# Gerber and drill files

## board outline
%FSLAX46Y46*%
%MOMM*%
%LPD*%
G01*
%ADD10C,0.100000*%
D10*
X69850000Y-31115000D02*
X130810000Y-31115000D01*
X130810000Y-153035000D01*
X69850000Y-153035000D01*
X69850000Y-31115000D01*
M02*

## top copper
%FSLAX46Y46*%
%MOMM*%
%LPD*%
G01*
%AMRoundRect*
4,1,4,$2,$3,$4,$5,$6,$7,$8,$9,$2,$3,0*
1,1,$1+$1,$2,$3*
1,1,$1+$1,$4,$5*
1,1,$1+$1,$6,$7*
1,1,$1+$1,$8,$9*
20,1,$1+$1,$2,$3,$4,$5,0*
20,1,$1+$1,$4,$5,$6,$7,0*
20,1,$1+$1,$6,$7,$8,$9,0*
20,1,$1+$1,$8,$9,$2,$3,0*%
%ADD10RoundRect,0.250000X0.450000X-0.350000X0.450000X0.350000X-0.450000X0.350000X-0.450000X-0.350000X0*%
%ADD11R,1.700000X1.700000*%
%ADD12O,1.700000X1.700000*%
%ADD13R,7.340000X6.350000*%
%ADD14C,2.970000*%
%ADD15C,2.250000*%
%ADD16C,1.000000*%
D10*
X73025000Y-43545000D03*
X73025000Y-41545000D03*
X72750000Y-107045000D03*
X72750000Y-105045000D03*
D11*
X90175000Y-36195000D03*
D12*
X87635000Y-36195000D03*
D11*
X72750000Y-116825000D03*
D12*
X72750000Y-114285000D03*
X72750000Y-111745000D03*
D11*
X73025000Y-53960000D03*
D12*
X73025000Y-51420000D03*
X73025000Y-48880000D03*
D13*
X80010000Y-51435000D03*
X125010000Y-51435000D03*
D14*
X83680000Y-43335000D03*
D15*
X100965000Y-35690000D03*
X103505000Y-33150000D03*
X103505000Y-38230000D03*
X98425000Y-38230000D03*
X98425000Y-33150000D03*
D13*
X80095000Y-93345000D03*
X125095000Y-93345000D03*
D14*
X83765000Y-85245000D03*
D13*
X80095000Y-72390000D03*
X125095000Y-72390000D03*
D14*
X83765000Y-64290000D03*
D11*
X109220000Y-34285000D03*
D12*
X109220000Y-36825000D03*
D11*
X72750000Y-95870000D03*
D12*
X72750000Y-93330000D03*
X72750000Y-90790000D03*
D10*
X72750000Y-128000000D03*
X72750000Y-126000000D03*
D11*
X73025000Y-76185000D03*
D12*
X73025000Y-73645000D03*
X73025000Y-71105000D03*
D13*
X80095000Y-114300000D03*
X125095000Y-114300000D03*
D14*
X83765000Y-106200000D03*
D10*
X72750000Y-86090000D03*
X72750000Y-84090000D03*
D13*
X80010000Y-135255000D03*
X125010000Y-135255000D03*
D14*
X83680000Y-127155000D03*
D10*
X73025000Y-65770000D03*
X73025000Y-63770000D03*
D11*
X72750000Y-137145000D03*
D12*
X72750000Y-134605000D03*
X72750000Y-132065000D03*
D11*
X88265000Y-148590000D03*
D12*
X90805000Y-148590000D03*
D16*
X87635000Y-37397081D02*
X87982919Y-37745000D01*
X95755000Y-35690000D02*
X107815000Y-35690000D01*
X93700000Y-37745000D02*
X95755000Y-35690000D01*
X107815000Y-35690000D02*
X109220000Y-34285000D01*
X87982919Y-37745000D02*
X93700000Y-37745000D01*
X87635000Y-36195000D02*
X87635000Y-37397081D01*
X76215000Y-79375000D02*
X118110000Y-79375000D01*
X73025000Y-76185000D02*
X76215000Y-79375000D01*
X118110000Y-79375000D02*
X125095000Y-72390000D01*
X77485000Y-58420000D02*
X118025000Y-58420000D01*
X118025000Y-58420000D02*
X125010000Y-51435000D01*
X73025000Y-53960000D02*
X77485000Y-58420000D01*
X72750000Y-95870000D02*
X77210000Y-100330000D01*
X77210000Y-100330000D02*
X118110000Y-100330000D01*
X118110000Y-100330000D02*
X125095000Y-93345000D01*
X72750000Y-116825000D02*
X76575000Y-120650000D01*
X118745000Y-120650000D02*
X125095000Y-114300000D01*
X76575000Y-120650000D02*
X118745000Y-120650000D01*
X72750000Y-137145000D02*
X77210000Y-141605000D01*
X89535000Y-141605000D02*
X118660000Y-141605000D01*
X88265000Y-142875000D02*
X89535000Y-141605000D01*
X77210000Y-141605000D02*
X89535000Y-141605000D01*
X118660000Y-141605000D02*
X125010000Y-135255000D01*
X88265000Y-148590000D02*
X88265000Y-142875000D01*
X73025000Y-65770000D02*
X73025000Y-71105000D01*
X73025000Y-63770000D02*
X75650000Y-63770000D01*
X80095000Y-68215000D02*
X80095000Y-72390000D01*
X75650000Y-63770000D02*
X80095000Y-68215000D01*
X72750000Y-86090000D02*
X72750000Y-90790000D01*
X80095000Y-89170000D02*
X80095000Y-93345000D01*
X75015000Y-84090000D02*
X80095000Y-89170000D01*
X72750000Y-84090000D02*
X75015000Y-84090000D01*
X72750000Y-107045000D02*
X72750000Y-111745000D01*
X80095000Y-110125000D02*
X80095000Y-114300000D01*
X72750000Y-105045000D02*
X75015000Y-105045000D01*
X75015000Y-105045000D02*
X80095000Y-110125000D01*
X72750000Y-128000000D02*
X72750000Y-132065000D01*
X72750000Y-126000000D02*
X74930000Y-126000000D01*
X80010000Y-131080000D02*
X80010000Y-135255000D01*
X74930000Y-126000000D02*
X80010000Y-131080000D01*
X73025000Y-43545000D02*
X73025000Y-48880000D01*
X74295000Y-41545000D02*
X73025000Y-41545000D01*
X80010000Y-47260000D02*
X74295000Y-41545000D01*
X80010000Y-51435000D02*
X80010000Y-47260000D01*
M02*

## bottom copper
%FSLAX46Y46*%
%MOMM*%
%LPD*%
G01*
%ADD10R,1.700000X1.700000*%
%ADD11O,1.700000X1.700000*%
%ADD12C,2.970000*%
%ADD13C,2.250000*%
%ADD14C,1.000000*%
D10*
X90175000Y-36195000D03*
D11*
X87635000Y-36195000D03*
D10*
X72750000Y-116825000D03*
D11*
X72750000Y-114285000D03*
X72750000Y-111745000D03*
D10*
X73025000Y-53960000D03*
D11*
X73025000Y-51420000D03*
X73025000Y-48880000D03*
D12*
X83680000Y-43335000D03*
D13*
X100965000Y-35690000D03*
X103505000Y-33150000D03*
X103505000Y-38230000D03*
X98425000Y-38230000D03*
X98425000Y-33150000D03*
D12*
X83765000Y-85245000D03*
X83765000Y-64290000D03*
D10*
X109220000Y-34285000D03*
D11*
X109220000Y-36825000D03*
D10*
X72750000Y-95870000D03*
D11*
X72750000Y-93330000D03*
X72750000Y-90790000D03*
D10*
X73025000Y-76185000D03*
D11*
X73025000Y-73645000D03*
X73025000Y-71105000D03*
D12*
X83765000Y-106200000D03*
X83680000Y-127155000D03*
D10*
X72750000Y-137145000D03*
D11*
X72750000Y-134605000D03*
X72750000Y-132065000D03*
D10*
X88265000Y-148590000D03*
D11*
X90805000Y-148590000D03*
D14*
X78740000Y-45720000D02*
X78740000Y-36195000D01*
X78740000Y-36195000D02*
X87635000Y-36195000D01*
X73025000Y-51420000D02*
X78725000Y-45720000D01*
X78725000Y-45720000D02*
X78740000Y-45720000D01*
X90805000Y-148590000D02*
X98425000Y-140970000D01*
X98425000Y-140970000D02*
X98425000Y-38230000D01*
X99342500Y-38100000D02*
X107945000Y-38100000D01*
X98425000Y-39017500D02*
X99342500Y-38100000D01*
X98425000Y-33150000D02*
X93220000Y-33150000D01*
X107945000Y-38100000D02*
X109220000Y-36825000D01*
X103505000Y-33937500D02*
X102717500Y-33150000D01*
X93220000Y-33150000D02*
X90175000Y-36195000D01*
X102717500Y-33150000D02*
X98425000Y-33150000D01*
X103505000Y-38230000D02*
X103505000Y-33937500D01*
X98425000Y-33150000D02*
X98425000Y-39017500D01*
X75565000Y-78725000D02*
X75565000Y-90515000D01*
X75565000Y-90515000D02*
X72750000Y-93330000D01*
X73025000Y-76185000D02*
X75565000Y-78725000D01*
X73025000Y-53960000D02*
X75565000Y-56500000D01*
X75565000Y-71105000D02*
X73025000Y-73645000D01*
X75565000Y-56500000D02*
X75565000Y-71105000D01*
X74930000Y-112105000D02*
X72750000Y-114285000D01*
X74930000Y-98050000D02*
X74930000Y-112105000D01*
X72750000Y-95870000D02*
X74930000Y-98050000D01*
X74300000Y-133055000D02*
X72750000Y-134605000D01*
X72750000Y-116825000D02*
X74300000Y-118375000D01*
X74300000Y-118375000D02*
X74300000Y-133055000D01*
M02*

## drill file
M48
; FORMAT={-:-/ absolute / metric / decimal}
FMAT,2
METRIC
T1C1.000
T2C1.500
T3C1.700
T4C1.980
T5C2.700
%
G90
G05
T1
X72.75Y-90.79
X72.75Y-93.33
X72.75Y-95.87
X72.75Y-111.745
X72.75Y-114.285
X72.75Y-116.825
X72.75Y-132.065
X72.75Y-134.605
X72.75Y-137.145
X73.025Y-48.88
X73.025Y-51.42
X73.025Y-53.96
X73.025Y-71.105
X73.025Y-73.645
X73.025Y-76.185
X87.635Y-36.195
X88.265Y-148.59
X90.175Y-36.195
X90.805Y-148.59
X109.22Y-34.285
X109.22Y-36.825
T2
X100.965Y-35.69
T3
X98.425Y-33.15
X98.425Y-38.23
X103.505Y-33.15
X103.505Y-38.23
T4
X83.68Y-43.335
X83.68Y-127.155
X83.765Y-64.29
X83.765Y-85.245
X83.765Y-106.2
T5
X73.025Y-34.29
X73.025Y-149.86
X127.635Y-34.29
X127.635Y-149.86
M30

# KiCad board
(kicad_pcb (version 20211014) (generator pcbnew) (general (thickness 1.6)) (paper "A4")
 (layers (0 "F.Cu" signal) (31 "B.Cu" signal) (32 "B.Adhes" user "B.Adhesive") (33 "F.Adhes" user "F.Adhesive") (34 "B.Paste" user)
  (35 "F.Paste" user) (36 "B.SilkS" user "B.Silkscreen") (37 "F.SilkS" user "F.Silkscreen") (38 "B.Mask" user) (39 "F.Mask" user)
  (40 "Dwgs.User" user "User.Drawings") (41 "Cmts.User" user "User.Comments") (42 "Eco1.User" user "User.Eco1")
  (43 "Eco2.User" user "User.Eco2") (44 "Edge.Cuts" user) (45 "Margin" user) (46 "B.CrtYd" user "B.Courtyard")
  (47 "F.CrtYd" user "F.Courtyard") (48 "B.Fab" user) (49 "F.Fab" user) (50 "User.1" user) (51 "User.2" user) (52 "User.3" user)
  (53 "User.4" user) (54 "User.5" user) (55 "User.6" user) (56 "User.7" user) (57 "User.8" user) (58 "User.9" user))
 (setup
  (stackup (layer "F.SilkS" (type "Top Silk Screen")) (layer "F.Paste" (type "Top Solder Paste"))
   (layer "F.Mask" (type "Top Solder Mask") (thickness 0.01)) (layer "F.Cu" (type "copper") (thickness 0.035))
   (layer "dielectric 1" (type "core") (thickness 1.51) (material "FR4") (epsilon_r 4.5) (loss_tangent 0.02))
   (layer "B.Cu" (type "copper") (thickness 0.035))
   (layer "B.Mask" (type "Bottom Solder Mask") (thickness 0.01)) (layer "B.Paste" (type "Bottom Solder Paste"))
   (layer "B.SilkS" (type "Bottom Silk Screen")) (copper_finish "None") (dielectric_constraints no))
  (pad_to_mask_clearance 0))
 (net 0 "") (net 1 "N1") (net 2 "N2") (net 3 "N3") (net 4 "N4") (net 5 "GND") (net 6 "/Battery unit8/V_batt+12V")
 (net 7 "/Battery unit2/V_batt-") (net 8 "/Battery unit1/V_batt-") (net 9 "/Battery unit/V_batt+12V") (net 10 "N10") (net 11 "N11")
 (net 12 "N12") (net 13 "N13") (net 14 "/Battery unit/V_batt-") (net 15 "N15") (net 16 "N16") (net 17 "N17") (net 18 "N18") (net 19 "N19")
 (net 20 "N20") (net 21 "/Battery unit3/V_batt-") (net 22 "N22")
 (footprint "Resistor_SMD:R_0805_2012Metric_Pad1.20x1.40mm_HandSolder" (layer "F.Cu") (at 73.025 42.545 90)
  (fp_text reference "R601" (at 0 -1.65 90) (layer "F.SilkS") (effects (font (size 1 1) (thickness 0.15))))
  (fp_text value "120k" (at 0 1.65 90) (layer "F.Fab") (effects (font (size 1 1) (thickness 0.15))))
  (pad "1" smd roundrect (at -1 0 90) (size 1.2 1.4) (layers "F.Cu" "F.Paste" "F.Mask") (roundrect_rratio 0.208333) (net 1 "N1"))
  (pad "2" smd roundrect (at 1 0 90) (size 1.2 1.4) (layers "F.Cu" "F.Paste" "F.Mask") (roundrect_rratio 0.208333) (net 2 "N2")))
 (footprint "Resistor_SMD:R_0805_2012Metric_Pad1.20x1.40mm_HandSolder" (layer "F.Cu") (at 72.75 106.045 90)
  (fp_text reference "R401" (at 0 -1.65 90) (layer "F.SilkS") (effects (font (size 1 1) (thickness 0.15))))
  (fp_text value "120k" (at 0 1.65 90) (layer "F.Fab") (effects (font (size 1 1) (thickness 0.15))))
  (pad "1" smd roundrect (at -1 0 90) (size 1.2 1.4) (layers "F.Cu" "F.Paste" "F.Mask") (roundrect_rratio 0.208333) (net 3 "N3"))
  (pad "2" smd roundrect (at 1 0 90) (size 1.2 1.4) (layers "F.Cu" "F.Paste" "F.Mask") (roundrect_rratio 0.208333) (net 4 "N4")))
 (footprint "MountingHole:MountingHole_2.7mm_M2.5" (layer "F.Cu") (at 127.635 149.86 180)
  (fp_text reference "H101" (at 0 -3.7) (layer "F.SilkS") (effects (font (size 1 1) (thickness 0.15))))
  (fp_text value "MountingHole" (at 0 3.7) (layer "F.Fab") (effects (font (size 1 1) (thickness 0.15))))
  (pad "" np_thru_hole circle (at 0 0 180) (size 2.7 2.7) (drill 2.7) (layers *.Cu *.Mask)))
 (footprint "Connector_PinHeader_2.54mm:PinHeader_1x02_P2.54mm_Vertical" (layer "F.Cu") (at 90.175 36.195 -90)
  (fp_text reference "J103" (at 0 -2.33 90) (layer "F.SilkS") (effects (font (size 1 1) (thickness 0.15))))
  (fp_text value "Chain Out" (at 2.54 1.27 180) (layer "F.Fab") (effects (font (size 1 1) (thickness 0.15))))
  (pad "1" thru_hole rect (at 0 0 270) (size 1.7 1.7) (drill 1) (layers *.Cu *.Mask) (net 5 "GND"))
  (pad "2" thru_hole oval (at 0 2.54 270) (size 1.7 1.7) (drill 1) (layers *.Cu *.Mask) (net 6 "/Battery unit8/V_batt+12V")))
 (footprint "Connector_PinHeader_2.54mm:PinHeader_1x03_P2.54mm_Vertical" (layer "F.Cu") (at 72.75 116.825 180)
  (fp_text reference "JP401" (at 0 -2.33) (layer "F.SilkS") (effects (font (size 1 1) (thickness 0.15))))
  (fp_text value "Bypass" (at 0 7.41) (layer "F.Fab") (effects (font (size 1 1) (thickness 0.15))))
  (pad "1" thru_hole rect (at 0 0 180) (size 1.7 1.7) (drill 1) (layers *.Cu *.Mask) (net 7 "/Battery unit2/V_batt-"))
  (pad "2" thru_hole oval (at 0 2.54 180) (size 1.7 1.7) (drill 1) (layers *.Cu *.Mask) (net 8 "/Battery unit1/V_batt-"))
  (pad "3" thru_hole oval (at 0 5.08 180) (size 1.7 1.7) (drill 1) (layers *.Cu *.Mask) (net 3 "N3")))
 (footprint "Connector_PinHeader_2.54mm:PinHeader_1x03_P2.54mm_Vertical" (layer "F.Cu") (at 73.025 53.96 180)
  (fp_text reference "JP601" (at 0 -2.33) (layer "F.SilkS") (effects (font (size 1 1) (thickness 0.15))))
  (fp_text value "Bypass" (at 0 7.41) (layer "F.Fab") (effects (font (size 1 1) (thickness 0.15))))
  (pad "1" thru_hole rect (at 0 0 180) (size 1.7 1.7) (drill 1) (layers *.Cu *.Mask) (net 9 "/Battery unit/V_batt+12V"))
  (pad "2" thru_hole oval (at 0 2.54 180) (size 1.7 1.7) (drill 1) (layers *.Cu *.Mask) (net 6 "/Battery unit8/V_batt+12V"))
  (pad "3" thru_hole oval (at 0 5.08 180) (size 1.7 1.7) (drill 1) (layers *.Cu *.Mask) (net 1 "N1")))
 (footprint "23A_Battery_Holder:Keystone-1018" (layer "F.Cu") (at 102.51 51.435)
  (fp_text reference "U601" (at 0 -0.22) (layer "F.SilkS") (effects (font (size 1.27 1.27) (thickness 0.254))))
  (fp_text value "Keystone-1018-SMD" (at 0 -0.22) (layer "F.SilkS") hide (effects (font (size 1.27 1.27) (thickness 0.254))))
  (pad "1" smd rect (at -22.5 0 90) (size 6.35 7.34) (layers "F.Cu" "F.Paste" "F.Mask") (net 2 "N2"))
  (pad "2" smd rect (at 22.5 0 90) (size 6.35 7.34) (layers "F.Cu" "F.Paste" "F.Mask") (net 9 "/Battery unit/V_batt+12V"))
  (pad "MH1" thru_hole circle (at -18.83 -8.1) (size 2.97 2.97) (drill 1.98) (layers *.Cu *.Mask) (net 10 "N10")))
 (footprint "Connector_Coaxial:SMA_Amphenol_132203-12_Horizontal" (layer "F.Cu") (at 100.965 35.69)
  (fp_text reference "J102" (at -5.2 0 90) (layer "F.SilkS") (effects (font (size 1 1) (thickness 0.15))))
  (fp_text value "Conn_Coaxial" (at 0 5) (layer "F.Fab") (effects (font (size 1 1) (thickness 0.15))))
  (pad "1" thru_hole circle (at 0 0) (size 2.25 2.25) (drill 1.5) (layers *.Cu *.Mask) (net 6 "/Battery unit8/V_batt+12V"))
  (pad "2" thru_hole circle (at 2.54 -2.54) (size 2.25 2.25) (drill 1.7) (layers *.Cu *.Mask) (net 5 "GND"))
  (pad "2" thru_hole circle (at 2.54 2.54 90) (size 2.25 2.25) (drill 1.7) (layers *.Cu *.Mask) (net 5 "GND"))
  (pad "2" thru_hole circle (at -2.54 2.54) (size 2.25 2.25) (drill 1.7) (layers *.Cu *.Mask) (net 5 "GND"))
  (pad "2" thru_hole circle (at -2.54 -2.54) (size 2.25 2.25) (drill 1.7) (layers *.Cu *.Mask) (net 5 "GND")))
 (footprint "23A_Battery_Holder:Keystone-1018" (layer "F.Cu") (at 102.595 93.345)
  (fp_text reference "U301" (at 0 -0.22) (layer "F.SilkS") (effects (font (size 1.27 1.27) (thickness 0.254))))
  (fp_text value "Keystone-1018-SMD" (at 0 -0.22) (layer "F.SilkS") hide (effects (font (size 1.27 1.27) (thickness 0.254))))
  (pad "1" smd rect (at -22.5 0 90) (size 6.35 7.34) (layers "F.Cu" "F.Paste" "F.Mask") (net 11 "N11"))
  (pad "2" smd rect (at 22.5 0 90) (size 6.35 7.34) (layers "F.Cu" "F.Paste" "F.Mask") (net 8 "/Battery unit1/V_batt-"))
  (pad "MH1" thru_hole circle (at -18.83 -8.1) (size 2.97 2.97) (drill 1.98) (layers *.Cu *.Mask) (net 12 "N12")))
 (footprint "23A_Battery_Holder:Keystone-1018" (layer "F.Cu") (at 102.595 72.39)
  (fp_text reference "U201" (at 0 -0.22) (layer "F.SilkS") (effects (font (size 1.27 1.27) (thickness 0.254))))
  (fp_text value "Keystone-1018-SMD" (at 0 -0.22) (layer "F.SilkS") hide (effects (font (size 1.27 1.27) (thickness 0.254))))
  (pad "1" smd rect (at -22.5 0 90) (size 6.35 7.34) (layers "F.Cu" "F.Paste" "F.Mask") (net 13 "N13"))
  (pad "2" smd rect (at 22.5 0 90) (size 6.35 7.34) (layers "F.Cu" "F.Paste" "F.Mask") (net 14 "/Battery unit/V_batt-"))
  (pad "MH1" thru_hole circle (at -18.83 -8.1) (size 2.97 2.97) (drill 1.98) (layers *.Cu *.Mask) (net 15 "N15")))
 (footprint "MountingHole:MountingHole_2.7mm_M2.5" (layer "F.Cu") (at 73.025 34.29)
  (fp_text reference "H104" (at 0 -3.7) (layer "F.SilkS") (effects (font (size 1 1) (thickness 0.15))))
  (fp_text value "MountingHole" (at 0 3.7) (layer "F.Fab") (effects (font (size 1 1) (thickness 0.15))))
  (pad "" np_thru_hole circle (at 0 0) (size 2.7 2.7) (drill 2.7) (layers *.Cu *.Mask)))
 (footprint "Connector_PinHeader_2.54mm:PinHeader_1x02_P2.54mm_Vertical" (layer "F.Cu") (at 109.22 34.285)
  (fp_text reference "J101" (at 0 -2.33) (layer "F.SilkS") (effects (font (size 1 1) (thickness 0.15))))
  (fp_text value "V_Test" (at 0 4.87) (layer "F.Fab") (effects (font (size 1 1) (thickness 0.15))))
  (pad "1" thru_hole rect (at 0 0) (size 1.7 1.7) (drill 1) (layers *.Cu *.Mask) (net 6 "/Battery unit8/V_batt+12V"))
  (pad "2" thru_hole oval (at 0 2.54) (size 1.7 1.7) (drill 1) (layers *.Cu *.Mask) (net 5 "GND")))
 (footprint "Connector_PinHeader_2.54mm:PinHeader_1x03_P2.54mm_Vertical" (layer "F.Cu") (at 72.75 95.87 180)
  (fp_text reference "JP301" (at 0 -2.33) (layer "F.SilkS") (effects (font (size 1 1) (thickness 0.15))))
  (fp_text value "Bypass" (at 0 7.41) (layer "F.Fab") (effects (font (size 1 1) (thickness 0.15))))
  (pad "1" thru_hole rect (at 0 0 180) (size 1.7 1.7) (drill 1) (layers *.Cu *.Mask) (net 8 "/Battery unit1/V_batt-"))
  (pad "2" thru_hole oval (at 0 2.54 180) (size 1.7 1.7) (drill 1) (layers *.Cu *.Mask) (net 14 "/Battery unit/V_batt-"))
  (pad "3" thru_hole oval (at 0 5.08 180) (size 1.7 1.7) (drill 1) (layers *.Cu *.Mask) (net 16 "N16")))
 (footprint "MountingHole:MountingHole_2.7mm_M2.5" (layer "F.Cu") (at 73.025 149.86)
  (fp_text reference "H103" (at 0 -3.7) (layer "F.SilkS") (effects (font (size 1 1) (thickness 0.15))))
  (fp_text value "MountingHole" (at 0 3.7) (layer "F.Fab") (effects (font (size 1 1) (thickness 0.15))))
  (pad "" np_thru_hole circle (at 0 0) (size 2.7 2.7) (drill 2.7) (layers *.Cu *.Mask)))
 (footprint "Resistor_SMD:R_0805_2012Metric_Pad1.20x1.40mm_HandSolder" (layer "F.Cu") (at 72.75 127 90)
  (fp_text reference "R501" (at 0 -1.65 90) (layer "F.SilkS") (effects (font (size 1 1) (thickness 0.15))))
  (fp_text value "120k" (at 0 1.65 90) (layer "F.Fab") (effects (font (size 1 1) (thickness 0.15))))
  (pad "1" smd roundrect (at -1 0 90) (size 1.2 1.4) (layers "F.Cu" "F.Paste" "F.Mask") (roundrect_rratio 0.208333) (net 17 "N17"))
  (pad "2" smd roundrect (at 1 0 90) (size 1.2 1.4) (layers "F.Cu" "F.Paste" "F.Mask") (roundrect_rratio 0.208333) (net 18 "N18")))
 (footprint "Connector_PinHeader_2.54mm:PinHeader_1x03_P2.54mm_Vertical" (layer "F.Cu") (at 73.025 76.185 180)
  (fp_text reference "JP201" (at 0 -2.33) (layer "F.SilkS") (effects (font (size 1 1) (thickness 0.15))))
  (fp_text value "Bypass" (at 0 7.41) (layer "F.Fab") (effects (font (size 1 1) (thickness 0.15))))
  (pad "1" thru_hole rect (at 0 0 180) (size 1.7 1.7) (drill 1) (layers *.Cu *.Mask) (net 14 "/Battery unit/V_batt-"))
  (pad "2" thru_hole oval (at 0 2.54 180) (size 1.7 1.7) (drill 1) (layers *.Cu *.Mask) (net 9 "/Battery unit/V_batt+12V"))
  (pad "3" thru_hole oval (at 0 5.08 180) (size 1.7 1.7) (drill 1) (layers *.Cu *.Mask) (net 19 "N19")))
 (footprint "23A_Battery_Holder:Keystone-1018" (layer "F.Cu") (at 102.595 114.3)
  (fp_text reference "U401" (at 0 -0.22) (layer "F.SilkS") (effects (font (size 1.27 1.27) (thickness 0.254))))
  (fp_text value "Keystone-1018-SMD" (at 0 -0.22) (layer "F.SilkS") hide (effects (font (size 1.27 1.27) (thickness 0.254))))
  (pad "1" smd rect (at -22.5 0 90) (size 6.35 7.34) (layers "F.Cu" "F.Paste" "F.Mask") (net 4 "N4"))
  (pad "2" smd rect (at 22.5 0 90) (size 6.35 7.34) (layers "F.Cu" "F.Paste" "F.Mask") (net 7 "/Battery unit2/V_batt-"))
  (pad "MH1" thru_hole circle (at -18.83 -8.1) (size 2.97 2.97) (drill 1.98) (layers *.Cu *.Mask) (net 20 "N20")))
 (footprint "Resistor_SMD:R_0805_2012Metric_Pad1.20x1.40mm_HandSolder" (layer "F.Cu") (at 72.75 85.09 90)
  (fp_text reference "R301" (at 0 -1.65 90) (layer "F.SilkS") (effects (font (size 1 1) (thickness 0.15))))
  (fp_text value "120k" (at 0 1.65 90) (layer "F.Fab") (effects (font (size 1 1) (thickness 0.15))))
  (pad "1" smd roundrect (at -1 0 90) (size 1.2 1.4) (layers "F.Cu" "F.Paste" "F.Mask") (roundrect_rratio 0.208333) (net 16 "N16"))
  (pad "2" smd roundrect (at 1 0 90) (size 1.2 1.4) (layers "F.Cu" "F.Paste" "F.Mask") (roundrect_rratio 0.208333) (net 11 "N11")))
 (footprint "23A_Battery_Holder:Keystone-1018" (layer "F.Cu") (at 102.51 135.255)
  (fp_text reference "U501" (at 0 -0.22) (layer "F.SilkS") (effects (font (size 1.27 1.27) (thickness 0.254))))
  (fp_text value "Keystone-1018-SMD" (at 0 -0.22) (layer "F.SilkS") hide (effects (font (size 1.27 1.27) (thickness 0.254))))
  (pad "1" smd rect (at -22.5 0 90) (size 6.35 7.34) (layers "F.Cu" "F.Paste" "F.Mask") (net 18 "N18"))
  (pad "2" smd rect (at 22.5 0 90) (size 6.35 7.34) (layers "F.Cu" "F.Paste" "F.Mask") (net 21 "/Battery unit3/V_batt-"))
  (pad "MH1" thru_hole circle (at -18.83 -8.1) (size 2.97 2.97) (drill 1.98) (layers *.Cu *.Mask) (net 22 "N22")))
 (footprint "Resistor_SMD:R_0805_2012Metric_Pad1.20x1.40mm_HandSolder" (layer "F.Cu") (at 73.025 64.77 90)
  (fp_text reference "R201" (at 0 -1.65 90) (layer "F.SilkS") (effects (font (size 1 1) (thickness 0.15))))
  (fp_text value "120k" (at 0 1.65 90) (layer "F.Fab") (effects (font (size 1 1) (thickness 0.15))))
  (pad "1" smd roundrect (at -1 0 90) (size 1.2 1.4) (layers "F.Cu" "F.Paste" "F.Mask") (roundrect_rratio 0.208333) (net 19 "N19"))
  (pad "2" smd roundrect (at 1 0 90) (size 1.2 1.4) (layers "F.Cu" "F.Paste" "F.Mask") (roundrect_rratio 0.208333) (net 13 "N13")))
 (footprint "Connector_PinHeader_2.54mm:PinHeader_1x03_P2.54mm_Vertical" (layer "F.Cu") (at 72.75 137.145 180)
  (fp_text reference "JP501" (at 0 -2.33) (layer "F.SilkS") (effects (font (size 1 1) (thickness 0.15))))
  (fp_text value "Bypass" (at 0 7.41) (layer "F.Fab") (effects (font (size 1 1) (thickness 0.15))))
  (pad "1" thru_hole rect (at 0 0 180) (size 1.7 1.7) (drill 1) (layers *.Cu *.Mask) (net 21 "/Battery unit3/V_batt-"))
  (pad "2" thru_hole oval (at 0 2.54 180) (size 1.7 1.7) (drill 1) (layers *.Cu *.Mask) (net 7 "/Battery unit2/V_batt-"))
  (pad "3" thru_hole oval (at 0 5.08 180) (size 1.7 1.7) (drill 1) (layers *.Cu *.Mask) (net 17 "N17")))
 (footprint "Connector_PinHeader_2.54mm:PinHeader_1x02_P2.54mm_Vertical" (layer "F.Cu") (at 88.265 148.59 90)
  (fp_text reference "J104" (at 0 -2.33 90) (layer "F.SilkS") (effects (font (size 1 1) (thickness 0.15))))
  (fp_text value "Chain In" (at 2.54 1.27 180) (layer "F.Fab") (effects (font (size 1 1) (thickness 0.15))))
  (pad "1" thru_hole rect (at 0 0 90) (size 1.7 1.7) (drill 1) (layers *.Cu *.Mask) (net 21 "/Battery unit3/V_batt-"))
  (pad "2" thru_hole oval (at 0 2.54 90) (size 1.7 1.7) (drill 1) (layers *.Cu *.Mask) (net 5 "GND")))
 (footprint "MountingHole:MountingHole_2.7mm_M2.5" (layer "F.Cu") (at 127.635 34.29 180)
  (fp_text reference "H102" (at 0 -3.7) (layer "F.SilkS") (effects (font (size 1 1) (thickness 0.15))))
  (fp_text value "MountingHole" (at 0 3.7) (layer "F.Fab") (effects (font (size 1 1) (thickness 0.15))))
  (pad "" np_thru_hole circle (at 0 0 180) (size 2.7 2.7) (drill 2.7) (layers *.Cu *.Mask)))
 (gr_rect (start 69.85 31.115) (end 130.81 153.035) (layer "Edge.Cuts") (width 0.1) (fill none))
 (segment (start 87.635 37.397081) (end 87.982919 37.745) (width 1) (layer "F.Cu") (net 6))
 (segment (start 95.755 35.69) (end 107.815 35.69) (width 1) (layer "F.Cu") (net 6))
 (segment (start 93.7 37.745) (end 95.755 35.69) (width 1) (layer "F.Cu") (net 6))
 (segment (start 107.815 35.69) (end 109.22 34.285) (width 1) (layer "F.Cu") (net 6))
 (segment (start 87.982919 37.745) (end 93.7 37.745) (width 1) (layer "F.Cu") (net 6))
 (segment (start 87.635 36.195) (end 87.635 37.397081) (width 1) (layer "F.Cu") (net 6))
 (segment (start 78.74 45.72) (end 78.74 36.195) (width 1) (layer "B.Cu") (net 6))
 (segment (start 78.74 36.195) (end 87.635 36.195) (width 1) (layer "B.Cu") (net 6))
 (segment (start 73.025 51.42) (end 78.725 45.72) (width 1) (layer "B.Cu") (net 6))
 (segment (start 78.725 45.72) (end 78.74 45.72) (width 1) (layer "B.Cu") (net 6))
 (segment (start 90.805 148.59) (end 98.425 140.97) (width 1) (layer "B.Cu") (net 5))
 (segment (start 98.425 140.97) (end 98.425 38.23) (width 1) (layer "B.Cu") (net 5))
 (segment (start 99.3425 38.1) (end 107.945 38.1) (width 1) (layer "B.Cu") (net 5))
 (segment (start 98.425 39.0175) (end 99.3425 38.1) (width 1) (layer "B.Cu") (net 5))
 (segment (start 98.425 33.15) (end 93.22 33.15) (width 1) (layer "B.Cu") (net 5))
 (segment (start 107.945 38.1) (end 109.22 36.825) (width 1) (layer "B.Cu") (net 5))
 (segment (start 103.505 33.9375) (end 102.7175 33.15) (width 1) (layer "B.Cu") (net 5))
 (segment (start 93.22 33.15) (end 90.175 36.195) (width 1) (layer "B.Cu") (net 5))
 (segment (start 102.7175 33.15) (end 98.425 33.15) (width 1) (layer "B.Cu") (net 5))
 (segment (start 103.505 38.23) (end 103.505 33.9375) (width 1) (layer "B.Cu") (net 5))
 (segment (start 98.425 33.15) (end 98.425 39.0175) (width 1) (layer "B.Cu") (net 5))
 (segment (start 76.215 79.375) (end 118.11 79.375) (width 1) (layer "F.Cu") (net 14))
 (segment (start 73.025 76.185) (end 76.215 79.375) (width 1) (layer "F.Cu") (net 14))
 (segment (start 118.11 79.375) (end 125.095 72.39) (width 1) (layer "F.Cu") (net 14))
 (segment (start 75.565 78.725) (end 75.565 90.515) (width 1) (layer "B.Cu") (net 14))
 (segment (start 75.565 90.515) (end 72.75 93.33) (width 1) (layer "B.Cu") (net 14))
 (segment (start 73.025 76.185) (end 75.565 78.725) (width 1) (layer "B.Cu") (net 14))
 (segment (start 77.485 58.42) (end 118.025 58.42) (width 1) (layer "F.Cu") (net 9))
 (segment (start 118.025 58.42) (end 125.01 51.435) (width 1) (layer "F.Cu") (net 9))
 (segment (start 73.025 53.96) (end 77.485 58.42) (width 1) (layer "F.Cu") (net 9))
 (segment (start 73.025 53.96) (end 75.565 56.5) (width 1) (layer "B.Cu") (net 9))
 (segment (start 75.565 71.105) (end 73.025 73.645) (width 1) (layer "B.Cu") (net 9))
 (segment (start 75.565 56.5) (end 75.565 71.105) (width 1) (layer "B.Cu") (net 9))
 (segment (start 72.75 95.87) (end 77.21 100.33) (width 1) (layer "F.Cu") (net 8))
 (segment (start 77.21 100.33) (end 118.11 100.33) (width 1) (layer "F.Cu") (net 8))
 (segment (start 118.11 100.33) (end 125.095 93.345) (width 1) (layer "F.Cu") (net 8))
 (segment (start 74.93 112.105) (end 72.75 114.285) (width 1) (layer "B.Cu") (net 8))
 (segment (start 74.93 98.05) (end 74.93 112.105) (width 1) (layer "B.Cu") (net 8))
 (segment (start 72.75 95.87) (end 74.93 98.05) (width 1) (layer "B.Cu") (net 8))
 (segment (start 72.75 116.825) (end 76.575 120.65) (width 1) (layer "F.Cu") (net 7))
 (segment (start 118.745 120.65) (end 125.095 114.3) (width 1) (layer "F.Cu") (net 7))
 (segment (start 76.575 120.65) (end 118.745 120.65) (width 1) (layer "F.Cu") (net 7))
 (segment (start 74.3 133.055) (end 72.75 134.605) (width 1) (layer "B.Cu") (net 7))
 (segment (start 72.75 116.825) (end 74.3 118.375) (width 1) (layer "B.Cu") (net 7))
 (segment (start 74.3 118.375) (end 74.3 133.055) (width 1) (layer "B.Cu") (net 7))
 (segment (start 72.75 137.145) (end 77.21 141.605) (width 1) (layer "F.Cu") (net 21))
 (segment (start 89.535 141.605) (end 118.66 141.605) (width 1) (layer "F.Cu") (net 21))
 (segment (start 88.265 142.875) (end 89.535 141.605) (width 1) (layer "F.Cu") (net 21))
 (segment (start 77.21 141.605) (end 89.535 141.605) (width 1) (layer "F.Cu") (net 21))
 (segment (start 118.66 141.605) (end 125.01 135.255) (width 1) (layer "F.Cu") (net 21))
 (segment (start 88.265 148.59) (end 88.265 142.875) (width 1) (layer "F.Cu") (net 21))
 (segment (start 73.025 65.77) (end 73.025 71.105) (width 1) (layer "F.Cu") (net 19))
 (segment (start 73.025 63.77) (end 75.65 63.77) (width 1) (layer "F.Cu") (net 13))
 (segment (start 80.095 68.215) (end 80.095 72.39) (width 1) (layer "F.Cu") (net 13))
 (segment (start 75.65 63.77) (end 80.095 68.215) (width 1) (layer "F.Cu") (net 13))
 (segment (start 72.75 86.09) (end 72.75 90.79) (width 1) (layer "F.Cu") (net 16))
 (segment (start 80.095 89.17) (end 80.095 93.345) (width 1) (layer "F.Cu") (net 11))
 (segment (start 75.015 84.09) (end 80.095 89.17) (width 1) (layer "F.Cu") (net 11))
 (segment (start 72.75 84.09) (end 75.015 84.09) (width 1) (layer "F.Cu") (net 11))
 (segment (start 72.75 107.045) (end 72.75 111.745) (width 1) (layer "F.Cu") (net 3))
 (segment (start 80.095 110.125) (end 80.095 114.3) (width 1) (layer "F.Cu") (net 4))
 (segment (start 72.75 105.045) (end 75.015 105.045) (width 1) (layer "F.Cu") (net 4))
 (segment (start 75.015 105.045) (end 80.095 110.125) (width 1) (layer "F.Cu") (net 4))
 (segment (start 72.75 128) (end 72.75 132.065) (width 1) (layer "F.Cu") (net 17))
 (segment (start 72.75 126) (end 74.93 126) (width 1) (layer "F.Cu") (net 18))
 (segment (start 80.01 131.08) (end 80.01 135.255) (width 1) (layer "F.Cu") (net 18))
 (segment (start 74.93 126) (end 80.01 131.08) (width 1) (layer "F.Cu") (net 18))
 (segment (start 73.025 43.545) (end 73.025 48.88) (width 1) (layer "F.Cu") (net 1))
 (segment (start 74.295 41.545) (end 73.025 41.545) (width 1) (layer "F.Cu") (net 2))
 (segment (start 80.01 47.26) (end 74.295 41.545) (width 1) (layer "F.Cu") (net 2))
 (segment (start 80.01 51.435) (end 80.01 47.26) (width 1) (layer "F.Cu") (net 2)))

